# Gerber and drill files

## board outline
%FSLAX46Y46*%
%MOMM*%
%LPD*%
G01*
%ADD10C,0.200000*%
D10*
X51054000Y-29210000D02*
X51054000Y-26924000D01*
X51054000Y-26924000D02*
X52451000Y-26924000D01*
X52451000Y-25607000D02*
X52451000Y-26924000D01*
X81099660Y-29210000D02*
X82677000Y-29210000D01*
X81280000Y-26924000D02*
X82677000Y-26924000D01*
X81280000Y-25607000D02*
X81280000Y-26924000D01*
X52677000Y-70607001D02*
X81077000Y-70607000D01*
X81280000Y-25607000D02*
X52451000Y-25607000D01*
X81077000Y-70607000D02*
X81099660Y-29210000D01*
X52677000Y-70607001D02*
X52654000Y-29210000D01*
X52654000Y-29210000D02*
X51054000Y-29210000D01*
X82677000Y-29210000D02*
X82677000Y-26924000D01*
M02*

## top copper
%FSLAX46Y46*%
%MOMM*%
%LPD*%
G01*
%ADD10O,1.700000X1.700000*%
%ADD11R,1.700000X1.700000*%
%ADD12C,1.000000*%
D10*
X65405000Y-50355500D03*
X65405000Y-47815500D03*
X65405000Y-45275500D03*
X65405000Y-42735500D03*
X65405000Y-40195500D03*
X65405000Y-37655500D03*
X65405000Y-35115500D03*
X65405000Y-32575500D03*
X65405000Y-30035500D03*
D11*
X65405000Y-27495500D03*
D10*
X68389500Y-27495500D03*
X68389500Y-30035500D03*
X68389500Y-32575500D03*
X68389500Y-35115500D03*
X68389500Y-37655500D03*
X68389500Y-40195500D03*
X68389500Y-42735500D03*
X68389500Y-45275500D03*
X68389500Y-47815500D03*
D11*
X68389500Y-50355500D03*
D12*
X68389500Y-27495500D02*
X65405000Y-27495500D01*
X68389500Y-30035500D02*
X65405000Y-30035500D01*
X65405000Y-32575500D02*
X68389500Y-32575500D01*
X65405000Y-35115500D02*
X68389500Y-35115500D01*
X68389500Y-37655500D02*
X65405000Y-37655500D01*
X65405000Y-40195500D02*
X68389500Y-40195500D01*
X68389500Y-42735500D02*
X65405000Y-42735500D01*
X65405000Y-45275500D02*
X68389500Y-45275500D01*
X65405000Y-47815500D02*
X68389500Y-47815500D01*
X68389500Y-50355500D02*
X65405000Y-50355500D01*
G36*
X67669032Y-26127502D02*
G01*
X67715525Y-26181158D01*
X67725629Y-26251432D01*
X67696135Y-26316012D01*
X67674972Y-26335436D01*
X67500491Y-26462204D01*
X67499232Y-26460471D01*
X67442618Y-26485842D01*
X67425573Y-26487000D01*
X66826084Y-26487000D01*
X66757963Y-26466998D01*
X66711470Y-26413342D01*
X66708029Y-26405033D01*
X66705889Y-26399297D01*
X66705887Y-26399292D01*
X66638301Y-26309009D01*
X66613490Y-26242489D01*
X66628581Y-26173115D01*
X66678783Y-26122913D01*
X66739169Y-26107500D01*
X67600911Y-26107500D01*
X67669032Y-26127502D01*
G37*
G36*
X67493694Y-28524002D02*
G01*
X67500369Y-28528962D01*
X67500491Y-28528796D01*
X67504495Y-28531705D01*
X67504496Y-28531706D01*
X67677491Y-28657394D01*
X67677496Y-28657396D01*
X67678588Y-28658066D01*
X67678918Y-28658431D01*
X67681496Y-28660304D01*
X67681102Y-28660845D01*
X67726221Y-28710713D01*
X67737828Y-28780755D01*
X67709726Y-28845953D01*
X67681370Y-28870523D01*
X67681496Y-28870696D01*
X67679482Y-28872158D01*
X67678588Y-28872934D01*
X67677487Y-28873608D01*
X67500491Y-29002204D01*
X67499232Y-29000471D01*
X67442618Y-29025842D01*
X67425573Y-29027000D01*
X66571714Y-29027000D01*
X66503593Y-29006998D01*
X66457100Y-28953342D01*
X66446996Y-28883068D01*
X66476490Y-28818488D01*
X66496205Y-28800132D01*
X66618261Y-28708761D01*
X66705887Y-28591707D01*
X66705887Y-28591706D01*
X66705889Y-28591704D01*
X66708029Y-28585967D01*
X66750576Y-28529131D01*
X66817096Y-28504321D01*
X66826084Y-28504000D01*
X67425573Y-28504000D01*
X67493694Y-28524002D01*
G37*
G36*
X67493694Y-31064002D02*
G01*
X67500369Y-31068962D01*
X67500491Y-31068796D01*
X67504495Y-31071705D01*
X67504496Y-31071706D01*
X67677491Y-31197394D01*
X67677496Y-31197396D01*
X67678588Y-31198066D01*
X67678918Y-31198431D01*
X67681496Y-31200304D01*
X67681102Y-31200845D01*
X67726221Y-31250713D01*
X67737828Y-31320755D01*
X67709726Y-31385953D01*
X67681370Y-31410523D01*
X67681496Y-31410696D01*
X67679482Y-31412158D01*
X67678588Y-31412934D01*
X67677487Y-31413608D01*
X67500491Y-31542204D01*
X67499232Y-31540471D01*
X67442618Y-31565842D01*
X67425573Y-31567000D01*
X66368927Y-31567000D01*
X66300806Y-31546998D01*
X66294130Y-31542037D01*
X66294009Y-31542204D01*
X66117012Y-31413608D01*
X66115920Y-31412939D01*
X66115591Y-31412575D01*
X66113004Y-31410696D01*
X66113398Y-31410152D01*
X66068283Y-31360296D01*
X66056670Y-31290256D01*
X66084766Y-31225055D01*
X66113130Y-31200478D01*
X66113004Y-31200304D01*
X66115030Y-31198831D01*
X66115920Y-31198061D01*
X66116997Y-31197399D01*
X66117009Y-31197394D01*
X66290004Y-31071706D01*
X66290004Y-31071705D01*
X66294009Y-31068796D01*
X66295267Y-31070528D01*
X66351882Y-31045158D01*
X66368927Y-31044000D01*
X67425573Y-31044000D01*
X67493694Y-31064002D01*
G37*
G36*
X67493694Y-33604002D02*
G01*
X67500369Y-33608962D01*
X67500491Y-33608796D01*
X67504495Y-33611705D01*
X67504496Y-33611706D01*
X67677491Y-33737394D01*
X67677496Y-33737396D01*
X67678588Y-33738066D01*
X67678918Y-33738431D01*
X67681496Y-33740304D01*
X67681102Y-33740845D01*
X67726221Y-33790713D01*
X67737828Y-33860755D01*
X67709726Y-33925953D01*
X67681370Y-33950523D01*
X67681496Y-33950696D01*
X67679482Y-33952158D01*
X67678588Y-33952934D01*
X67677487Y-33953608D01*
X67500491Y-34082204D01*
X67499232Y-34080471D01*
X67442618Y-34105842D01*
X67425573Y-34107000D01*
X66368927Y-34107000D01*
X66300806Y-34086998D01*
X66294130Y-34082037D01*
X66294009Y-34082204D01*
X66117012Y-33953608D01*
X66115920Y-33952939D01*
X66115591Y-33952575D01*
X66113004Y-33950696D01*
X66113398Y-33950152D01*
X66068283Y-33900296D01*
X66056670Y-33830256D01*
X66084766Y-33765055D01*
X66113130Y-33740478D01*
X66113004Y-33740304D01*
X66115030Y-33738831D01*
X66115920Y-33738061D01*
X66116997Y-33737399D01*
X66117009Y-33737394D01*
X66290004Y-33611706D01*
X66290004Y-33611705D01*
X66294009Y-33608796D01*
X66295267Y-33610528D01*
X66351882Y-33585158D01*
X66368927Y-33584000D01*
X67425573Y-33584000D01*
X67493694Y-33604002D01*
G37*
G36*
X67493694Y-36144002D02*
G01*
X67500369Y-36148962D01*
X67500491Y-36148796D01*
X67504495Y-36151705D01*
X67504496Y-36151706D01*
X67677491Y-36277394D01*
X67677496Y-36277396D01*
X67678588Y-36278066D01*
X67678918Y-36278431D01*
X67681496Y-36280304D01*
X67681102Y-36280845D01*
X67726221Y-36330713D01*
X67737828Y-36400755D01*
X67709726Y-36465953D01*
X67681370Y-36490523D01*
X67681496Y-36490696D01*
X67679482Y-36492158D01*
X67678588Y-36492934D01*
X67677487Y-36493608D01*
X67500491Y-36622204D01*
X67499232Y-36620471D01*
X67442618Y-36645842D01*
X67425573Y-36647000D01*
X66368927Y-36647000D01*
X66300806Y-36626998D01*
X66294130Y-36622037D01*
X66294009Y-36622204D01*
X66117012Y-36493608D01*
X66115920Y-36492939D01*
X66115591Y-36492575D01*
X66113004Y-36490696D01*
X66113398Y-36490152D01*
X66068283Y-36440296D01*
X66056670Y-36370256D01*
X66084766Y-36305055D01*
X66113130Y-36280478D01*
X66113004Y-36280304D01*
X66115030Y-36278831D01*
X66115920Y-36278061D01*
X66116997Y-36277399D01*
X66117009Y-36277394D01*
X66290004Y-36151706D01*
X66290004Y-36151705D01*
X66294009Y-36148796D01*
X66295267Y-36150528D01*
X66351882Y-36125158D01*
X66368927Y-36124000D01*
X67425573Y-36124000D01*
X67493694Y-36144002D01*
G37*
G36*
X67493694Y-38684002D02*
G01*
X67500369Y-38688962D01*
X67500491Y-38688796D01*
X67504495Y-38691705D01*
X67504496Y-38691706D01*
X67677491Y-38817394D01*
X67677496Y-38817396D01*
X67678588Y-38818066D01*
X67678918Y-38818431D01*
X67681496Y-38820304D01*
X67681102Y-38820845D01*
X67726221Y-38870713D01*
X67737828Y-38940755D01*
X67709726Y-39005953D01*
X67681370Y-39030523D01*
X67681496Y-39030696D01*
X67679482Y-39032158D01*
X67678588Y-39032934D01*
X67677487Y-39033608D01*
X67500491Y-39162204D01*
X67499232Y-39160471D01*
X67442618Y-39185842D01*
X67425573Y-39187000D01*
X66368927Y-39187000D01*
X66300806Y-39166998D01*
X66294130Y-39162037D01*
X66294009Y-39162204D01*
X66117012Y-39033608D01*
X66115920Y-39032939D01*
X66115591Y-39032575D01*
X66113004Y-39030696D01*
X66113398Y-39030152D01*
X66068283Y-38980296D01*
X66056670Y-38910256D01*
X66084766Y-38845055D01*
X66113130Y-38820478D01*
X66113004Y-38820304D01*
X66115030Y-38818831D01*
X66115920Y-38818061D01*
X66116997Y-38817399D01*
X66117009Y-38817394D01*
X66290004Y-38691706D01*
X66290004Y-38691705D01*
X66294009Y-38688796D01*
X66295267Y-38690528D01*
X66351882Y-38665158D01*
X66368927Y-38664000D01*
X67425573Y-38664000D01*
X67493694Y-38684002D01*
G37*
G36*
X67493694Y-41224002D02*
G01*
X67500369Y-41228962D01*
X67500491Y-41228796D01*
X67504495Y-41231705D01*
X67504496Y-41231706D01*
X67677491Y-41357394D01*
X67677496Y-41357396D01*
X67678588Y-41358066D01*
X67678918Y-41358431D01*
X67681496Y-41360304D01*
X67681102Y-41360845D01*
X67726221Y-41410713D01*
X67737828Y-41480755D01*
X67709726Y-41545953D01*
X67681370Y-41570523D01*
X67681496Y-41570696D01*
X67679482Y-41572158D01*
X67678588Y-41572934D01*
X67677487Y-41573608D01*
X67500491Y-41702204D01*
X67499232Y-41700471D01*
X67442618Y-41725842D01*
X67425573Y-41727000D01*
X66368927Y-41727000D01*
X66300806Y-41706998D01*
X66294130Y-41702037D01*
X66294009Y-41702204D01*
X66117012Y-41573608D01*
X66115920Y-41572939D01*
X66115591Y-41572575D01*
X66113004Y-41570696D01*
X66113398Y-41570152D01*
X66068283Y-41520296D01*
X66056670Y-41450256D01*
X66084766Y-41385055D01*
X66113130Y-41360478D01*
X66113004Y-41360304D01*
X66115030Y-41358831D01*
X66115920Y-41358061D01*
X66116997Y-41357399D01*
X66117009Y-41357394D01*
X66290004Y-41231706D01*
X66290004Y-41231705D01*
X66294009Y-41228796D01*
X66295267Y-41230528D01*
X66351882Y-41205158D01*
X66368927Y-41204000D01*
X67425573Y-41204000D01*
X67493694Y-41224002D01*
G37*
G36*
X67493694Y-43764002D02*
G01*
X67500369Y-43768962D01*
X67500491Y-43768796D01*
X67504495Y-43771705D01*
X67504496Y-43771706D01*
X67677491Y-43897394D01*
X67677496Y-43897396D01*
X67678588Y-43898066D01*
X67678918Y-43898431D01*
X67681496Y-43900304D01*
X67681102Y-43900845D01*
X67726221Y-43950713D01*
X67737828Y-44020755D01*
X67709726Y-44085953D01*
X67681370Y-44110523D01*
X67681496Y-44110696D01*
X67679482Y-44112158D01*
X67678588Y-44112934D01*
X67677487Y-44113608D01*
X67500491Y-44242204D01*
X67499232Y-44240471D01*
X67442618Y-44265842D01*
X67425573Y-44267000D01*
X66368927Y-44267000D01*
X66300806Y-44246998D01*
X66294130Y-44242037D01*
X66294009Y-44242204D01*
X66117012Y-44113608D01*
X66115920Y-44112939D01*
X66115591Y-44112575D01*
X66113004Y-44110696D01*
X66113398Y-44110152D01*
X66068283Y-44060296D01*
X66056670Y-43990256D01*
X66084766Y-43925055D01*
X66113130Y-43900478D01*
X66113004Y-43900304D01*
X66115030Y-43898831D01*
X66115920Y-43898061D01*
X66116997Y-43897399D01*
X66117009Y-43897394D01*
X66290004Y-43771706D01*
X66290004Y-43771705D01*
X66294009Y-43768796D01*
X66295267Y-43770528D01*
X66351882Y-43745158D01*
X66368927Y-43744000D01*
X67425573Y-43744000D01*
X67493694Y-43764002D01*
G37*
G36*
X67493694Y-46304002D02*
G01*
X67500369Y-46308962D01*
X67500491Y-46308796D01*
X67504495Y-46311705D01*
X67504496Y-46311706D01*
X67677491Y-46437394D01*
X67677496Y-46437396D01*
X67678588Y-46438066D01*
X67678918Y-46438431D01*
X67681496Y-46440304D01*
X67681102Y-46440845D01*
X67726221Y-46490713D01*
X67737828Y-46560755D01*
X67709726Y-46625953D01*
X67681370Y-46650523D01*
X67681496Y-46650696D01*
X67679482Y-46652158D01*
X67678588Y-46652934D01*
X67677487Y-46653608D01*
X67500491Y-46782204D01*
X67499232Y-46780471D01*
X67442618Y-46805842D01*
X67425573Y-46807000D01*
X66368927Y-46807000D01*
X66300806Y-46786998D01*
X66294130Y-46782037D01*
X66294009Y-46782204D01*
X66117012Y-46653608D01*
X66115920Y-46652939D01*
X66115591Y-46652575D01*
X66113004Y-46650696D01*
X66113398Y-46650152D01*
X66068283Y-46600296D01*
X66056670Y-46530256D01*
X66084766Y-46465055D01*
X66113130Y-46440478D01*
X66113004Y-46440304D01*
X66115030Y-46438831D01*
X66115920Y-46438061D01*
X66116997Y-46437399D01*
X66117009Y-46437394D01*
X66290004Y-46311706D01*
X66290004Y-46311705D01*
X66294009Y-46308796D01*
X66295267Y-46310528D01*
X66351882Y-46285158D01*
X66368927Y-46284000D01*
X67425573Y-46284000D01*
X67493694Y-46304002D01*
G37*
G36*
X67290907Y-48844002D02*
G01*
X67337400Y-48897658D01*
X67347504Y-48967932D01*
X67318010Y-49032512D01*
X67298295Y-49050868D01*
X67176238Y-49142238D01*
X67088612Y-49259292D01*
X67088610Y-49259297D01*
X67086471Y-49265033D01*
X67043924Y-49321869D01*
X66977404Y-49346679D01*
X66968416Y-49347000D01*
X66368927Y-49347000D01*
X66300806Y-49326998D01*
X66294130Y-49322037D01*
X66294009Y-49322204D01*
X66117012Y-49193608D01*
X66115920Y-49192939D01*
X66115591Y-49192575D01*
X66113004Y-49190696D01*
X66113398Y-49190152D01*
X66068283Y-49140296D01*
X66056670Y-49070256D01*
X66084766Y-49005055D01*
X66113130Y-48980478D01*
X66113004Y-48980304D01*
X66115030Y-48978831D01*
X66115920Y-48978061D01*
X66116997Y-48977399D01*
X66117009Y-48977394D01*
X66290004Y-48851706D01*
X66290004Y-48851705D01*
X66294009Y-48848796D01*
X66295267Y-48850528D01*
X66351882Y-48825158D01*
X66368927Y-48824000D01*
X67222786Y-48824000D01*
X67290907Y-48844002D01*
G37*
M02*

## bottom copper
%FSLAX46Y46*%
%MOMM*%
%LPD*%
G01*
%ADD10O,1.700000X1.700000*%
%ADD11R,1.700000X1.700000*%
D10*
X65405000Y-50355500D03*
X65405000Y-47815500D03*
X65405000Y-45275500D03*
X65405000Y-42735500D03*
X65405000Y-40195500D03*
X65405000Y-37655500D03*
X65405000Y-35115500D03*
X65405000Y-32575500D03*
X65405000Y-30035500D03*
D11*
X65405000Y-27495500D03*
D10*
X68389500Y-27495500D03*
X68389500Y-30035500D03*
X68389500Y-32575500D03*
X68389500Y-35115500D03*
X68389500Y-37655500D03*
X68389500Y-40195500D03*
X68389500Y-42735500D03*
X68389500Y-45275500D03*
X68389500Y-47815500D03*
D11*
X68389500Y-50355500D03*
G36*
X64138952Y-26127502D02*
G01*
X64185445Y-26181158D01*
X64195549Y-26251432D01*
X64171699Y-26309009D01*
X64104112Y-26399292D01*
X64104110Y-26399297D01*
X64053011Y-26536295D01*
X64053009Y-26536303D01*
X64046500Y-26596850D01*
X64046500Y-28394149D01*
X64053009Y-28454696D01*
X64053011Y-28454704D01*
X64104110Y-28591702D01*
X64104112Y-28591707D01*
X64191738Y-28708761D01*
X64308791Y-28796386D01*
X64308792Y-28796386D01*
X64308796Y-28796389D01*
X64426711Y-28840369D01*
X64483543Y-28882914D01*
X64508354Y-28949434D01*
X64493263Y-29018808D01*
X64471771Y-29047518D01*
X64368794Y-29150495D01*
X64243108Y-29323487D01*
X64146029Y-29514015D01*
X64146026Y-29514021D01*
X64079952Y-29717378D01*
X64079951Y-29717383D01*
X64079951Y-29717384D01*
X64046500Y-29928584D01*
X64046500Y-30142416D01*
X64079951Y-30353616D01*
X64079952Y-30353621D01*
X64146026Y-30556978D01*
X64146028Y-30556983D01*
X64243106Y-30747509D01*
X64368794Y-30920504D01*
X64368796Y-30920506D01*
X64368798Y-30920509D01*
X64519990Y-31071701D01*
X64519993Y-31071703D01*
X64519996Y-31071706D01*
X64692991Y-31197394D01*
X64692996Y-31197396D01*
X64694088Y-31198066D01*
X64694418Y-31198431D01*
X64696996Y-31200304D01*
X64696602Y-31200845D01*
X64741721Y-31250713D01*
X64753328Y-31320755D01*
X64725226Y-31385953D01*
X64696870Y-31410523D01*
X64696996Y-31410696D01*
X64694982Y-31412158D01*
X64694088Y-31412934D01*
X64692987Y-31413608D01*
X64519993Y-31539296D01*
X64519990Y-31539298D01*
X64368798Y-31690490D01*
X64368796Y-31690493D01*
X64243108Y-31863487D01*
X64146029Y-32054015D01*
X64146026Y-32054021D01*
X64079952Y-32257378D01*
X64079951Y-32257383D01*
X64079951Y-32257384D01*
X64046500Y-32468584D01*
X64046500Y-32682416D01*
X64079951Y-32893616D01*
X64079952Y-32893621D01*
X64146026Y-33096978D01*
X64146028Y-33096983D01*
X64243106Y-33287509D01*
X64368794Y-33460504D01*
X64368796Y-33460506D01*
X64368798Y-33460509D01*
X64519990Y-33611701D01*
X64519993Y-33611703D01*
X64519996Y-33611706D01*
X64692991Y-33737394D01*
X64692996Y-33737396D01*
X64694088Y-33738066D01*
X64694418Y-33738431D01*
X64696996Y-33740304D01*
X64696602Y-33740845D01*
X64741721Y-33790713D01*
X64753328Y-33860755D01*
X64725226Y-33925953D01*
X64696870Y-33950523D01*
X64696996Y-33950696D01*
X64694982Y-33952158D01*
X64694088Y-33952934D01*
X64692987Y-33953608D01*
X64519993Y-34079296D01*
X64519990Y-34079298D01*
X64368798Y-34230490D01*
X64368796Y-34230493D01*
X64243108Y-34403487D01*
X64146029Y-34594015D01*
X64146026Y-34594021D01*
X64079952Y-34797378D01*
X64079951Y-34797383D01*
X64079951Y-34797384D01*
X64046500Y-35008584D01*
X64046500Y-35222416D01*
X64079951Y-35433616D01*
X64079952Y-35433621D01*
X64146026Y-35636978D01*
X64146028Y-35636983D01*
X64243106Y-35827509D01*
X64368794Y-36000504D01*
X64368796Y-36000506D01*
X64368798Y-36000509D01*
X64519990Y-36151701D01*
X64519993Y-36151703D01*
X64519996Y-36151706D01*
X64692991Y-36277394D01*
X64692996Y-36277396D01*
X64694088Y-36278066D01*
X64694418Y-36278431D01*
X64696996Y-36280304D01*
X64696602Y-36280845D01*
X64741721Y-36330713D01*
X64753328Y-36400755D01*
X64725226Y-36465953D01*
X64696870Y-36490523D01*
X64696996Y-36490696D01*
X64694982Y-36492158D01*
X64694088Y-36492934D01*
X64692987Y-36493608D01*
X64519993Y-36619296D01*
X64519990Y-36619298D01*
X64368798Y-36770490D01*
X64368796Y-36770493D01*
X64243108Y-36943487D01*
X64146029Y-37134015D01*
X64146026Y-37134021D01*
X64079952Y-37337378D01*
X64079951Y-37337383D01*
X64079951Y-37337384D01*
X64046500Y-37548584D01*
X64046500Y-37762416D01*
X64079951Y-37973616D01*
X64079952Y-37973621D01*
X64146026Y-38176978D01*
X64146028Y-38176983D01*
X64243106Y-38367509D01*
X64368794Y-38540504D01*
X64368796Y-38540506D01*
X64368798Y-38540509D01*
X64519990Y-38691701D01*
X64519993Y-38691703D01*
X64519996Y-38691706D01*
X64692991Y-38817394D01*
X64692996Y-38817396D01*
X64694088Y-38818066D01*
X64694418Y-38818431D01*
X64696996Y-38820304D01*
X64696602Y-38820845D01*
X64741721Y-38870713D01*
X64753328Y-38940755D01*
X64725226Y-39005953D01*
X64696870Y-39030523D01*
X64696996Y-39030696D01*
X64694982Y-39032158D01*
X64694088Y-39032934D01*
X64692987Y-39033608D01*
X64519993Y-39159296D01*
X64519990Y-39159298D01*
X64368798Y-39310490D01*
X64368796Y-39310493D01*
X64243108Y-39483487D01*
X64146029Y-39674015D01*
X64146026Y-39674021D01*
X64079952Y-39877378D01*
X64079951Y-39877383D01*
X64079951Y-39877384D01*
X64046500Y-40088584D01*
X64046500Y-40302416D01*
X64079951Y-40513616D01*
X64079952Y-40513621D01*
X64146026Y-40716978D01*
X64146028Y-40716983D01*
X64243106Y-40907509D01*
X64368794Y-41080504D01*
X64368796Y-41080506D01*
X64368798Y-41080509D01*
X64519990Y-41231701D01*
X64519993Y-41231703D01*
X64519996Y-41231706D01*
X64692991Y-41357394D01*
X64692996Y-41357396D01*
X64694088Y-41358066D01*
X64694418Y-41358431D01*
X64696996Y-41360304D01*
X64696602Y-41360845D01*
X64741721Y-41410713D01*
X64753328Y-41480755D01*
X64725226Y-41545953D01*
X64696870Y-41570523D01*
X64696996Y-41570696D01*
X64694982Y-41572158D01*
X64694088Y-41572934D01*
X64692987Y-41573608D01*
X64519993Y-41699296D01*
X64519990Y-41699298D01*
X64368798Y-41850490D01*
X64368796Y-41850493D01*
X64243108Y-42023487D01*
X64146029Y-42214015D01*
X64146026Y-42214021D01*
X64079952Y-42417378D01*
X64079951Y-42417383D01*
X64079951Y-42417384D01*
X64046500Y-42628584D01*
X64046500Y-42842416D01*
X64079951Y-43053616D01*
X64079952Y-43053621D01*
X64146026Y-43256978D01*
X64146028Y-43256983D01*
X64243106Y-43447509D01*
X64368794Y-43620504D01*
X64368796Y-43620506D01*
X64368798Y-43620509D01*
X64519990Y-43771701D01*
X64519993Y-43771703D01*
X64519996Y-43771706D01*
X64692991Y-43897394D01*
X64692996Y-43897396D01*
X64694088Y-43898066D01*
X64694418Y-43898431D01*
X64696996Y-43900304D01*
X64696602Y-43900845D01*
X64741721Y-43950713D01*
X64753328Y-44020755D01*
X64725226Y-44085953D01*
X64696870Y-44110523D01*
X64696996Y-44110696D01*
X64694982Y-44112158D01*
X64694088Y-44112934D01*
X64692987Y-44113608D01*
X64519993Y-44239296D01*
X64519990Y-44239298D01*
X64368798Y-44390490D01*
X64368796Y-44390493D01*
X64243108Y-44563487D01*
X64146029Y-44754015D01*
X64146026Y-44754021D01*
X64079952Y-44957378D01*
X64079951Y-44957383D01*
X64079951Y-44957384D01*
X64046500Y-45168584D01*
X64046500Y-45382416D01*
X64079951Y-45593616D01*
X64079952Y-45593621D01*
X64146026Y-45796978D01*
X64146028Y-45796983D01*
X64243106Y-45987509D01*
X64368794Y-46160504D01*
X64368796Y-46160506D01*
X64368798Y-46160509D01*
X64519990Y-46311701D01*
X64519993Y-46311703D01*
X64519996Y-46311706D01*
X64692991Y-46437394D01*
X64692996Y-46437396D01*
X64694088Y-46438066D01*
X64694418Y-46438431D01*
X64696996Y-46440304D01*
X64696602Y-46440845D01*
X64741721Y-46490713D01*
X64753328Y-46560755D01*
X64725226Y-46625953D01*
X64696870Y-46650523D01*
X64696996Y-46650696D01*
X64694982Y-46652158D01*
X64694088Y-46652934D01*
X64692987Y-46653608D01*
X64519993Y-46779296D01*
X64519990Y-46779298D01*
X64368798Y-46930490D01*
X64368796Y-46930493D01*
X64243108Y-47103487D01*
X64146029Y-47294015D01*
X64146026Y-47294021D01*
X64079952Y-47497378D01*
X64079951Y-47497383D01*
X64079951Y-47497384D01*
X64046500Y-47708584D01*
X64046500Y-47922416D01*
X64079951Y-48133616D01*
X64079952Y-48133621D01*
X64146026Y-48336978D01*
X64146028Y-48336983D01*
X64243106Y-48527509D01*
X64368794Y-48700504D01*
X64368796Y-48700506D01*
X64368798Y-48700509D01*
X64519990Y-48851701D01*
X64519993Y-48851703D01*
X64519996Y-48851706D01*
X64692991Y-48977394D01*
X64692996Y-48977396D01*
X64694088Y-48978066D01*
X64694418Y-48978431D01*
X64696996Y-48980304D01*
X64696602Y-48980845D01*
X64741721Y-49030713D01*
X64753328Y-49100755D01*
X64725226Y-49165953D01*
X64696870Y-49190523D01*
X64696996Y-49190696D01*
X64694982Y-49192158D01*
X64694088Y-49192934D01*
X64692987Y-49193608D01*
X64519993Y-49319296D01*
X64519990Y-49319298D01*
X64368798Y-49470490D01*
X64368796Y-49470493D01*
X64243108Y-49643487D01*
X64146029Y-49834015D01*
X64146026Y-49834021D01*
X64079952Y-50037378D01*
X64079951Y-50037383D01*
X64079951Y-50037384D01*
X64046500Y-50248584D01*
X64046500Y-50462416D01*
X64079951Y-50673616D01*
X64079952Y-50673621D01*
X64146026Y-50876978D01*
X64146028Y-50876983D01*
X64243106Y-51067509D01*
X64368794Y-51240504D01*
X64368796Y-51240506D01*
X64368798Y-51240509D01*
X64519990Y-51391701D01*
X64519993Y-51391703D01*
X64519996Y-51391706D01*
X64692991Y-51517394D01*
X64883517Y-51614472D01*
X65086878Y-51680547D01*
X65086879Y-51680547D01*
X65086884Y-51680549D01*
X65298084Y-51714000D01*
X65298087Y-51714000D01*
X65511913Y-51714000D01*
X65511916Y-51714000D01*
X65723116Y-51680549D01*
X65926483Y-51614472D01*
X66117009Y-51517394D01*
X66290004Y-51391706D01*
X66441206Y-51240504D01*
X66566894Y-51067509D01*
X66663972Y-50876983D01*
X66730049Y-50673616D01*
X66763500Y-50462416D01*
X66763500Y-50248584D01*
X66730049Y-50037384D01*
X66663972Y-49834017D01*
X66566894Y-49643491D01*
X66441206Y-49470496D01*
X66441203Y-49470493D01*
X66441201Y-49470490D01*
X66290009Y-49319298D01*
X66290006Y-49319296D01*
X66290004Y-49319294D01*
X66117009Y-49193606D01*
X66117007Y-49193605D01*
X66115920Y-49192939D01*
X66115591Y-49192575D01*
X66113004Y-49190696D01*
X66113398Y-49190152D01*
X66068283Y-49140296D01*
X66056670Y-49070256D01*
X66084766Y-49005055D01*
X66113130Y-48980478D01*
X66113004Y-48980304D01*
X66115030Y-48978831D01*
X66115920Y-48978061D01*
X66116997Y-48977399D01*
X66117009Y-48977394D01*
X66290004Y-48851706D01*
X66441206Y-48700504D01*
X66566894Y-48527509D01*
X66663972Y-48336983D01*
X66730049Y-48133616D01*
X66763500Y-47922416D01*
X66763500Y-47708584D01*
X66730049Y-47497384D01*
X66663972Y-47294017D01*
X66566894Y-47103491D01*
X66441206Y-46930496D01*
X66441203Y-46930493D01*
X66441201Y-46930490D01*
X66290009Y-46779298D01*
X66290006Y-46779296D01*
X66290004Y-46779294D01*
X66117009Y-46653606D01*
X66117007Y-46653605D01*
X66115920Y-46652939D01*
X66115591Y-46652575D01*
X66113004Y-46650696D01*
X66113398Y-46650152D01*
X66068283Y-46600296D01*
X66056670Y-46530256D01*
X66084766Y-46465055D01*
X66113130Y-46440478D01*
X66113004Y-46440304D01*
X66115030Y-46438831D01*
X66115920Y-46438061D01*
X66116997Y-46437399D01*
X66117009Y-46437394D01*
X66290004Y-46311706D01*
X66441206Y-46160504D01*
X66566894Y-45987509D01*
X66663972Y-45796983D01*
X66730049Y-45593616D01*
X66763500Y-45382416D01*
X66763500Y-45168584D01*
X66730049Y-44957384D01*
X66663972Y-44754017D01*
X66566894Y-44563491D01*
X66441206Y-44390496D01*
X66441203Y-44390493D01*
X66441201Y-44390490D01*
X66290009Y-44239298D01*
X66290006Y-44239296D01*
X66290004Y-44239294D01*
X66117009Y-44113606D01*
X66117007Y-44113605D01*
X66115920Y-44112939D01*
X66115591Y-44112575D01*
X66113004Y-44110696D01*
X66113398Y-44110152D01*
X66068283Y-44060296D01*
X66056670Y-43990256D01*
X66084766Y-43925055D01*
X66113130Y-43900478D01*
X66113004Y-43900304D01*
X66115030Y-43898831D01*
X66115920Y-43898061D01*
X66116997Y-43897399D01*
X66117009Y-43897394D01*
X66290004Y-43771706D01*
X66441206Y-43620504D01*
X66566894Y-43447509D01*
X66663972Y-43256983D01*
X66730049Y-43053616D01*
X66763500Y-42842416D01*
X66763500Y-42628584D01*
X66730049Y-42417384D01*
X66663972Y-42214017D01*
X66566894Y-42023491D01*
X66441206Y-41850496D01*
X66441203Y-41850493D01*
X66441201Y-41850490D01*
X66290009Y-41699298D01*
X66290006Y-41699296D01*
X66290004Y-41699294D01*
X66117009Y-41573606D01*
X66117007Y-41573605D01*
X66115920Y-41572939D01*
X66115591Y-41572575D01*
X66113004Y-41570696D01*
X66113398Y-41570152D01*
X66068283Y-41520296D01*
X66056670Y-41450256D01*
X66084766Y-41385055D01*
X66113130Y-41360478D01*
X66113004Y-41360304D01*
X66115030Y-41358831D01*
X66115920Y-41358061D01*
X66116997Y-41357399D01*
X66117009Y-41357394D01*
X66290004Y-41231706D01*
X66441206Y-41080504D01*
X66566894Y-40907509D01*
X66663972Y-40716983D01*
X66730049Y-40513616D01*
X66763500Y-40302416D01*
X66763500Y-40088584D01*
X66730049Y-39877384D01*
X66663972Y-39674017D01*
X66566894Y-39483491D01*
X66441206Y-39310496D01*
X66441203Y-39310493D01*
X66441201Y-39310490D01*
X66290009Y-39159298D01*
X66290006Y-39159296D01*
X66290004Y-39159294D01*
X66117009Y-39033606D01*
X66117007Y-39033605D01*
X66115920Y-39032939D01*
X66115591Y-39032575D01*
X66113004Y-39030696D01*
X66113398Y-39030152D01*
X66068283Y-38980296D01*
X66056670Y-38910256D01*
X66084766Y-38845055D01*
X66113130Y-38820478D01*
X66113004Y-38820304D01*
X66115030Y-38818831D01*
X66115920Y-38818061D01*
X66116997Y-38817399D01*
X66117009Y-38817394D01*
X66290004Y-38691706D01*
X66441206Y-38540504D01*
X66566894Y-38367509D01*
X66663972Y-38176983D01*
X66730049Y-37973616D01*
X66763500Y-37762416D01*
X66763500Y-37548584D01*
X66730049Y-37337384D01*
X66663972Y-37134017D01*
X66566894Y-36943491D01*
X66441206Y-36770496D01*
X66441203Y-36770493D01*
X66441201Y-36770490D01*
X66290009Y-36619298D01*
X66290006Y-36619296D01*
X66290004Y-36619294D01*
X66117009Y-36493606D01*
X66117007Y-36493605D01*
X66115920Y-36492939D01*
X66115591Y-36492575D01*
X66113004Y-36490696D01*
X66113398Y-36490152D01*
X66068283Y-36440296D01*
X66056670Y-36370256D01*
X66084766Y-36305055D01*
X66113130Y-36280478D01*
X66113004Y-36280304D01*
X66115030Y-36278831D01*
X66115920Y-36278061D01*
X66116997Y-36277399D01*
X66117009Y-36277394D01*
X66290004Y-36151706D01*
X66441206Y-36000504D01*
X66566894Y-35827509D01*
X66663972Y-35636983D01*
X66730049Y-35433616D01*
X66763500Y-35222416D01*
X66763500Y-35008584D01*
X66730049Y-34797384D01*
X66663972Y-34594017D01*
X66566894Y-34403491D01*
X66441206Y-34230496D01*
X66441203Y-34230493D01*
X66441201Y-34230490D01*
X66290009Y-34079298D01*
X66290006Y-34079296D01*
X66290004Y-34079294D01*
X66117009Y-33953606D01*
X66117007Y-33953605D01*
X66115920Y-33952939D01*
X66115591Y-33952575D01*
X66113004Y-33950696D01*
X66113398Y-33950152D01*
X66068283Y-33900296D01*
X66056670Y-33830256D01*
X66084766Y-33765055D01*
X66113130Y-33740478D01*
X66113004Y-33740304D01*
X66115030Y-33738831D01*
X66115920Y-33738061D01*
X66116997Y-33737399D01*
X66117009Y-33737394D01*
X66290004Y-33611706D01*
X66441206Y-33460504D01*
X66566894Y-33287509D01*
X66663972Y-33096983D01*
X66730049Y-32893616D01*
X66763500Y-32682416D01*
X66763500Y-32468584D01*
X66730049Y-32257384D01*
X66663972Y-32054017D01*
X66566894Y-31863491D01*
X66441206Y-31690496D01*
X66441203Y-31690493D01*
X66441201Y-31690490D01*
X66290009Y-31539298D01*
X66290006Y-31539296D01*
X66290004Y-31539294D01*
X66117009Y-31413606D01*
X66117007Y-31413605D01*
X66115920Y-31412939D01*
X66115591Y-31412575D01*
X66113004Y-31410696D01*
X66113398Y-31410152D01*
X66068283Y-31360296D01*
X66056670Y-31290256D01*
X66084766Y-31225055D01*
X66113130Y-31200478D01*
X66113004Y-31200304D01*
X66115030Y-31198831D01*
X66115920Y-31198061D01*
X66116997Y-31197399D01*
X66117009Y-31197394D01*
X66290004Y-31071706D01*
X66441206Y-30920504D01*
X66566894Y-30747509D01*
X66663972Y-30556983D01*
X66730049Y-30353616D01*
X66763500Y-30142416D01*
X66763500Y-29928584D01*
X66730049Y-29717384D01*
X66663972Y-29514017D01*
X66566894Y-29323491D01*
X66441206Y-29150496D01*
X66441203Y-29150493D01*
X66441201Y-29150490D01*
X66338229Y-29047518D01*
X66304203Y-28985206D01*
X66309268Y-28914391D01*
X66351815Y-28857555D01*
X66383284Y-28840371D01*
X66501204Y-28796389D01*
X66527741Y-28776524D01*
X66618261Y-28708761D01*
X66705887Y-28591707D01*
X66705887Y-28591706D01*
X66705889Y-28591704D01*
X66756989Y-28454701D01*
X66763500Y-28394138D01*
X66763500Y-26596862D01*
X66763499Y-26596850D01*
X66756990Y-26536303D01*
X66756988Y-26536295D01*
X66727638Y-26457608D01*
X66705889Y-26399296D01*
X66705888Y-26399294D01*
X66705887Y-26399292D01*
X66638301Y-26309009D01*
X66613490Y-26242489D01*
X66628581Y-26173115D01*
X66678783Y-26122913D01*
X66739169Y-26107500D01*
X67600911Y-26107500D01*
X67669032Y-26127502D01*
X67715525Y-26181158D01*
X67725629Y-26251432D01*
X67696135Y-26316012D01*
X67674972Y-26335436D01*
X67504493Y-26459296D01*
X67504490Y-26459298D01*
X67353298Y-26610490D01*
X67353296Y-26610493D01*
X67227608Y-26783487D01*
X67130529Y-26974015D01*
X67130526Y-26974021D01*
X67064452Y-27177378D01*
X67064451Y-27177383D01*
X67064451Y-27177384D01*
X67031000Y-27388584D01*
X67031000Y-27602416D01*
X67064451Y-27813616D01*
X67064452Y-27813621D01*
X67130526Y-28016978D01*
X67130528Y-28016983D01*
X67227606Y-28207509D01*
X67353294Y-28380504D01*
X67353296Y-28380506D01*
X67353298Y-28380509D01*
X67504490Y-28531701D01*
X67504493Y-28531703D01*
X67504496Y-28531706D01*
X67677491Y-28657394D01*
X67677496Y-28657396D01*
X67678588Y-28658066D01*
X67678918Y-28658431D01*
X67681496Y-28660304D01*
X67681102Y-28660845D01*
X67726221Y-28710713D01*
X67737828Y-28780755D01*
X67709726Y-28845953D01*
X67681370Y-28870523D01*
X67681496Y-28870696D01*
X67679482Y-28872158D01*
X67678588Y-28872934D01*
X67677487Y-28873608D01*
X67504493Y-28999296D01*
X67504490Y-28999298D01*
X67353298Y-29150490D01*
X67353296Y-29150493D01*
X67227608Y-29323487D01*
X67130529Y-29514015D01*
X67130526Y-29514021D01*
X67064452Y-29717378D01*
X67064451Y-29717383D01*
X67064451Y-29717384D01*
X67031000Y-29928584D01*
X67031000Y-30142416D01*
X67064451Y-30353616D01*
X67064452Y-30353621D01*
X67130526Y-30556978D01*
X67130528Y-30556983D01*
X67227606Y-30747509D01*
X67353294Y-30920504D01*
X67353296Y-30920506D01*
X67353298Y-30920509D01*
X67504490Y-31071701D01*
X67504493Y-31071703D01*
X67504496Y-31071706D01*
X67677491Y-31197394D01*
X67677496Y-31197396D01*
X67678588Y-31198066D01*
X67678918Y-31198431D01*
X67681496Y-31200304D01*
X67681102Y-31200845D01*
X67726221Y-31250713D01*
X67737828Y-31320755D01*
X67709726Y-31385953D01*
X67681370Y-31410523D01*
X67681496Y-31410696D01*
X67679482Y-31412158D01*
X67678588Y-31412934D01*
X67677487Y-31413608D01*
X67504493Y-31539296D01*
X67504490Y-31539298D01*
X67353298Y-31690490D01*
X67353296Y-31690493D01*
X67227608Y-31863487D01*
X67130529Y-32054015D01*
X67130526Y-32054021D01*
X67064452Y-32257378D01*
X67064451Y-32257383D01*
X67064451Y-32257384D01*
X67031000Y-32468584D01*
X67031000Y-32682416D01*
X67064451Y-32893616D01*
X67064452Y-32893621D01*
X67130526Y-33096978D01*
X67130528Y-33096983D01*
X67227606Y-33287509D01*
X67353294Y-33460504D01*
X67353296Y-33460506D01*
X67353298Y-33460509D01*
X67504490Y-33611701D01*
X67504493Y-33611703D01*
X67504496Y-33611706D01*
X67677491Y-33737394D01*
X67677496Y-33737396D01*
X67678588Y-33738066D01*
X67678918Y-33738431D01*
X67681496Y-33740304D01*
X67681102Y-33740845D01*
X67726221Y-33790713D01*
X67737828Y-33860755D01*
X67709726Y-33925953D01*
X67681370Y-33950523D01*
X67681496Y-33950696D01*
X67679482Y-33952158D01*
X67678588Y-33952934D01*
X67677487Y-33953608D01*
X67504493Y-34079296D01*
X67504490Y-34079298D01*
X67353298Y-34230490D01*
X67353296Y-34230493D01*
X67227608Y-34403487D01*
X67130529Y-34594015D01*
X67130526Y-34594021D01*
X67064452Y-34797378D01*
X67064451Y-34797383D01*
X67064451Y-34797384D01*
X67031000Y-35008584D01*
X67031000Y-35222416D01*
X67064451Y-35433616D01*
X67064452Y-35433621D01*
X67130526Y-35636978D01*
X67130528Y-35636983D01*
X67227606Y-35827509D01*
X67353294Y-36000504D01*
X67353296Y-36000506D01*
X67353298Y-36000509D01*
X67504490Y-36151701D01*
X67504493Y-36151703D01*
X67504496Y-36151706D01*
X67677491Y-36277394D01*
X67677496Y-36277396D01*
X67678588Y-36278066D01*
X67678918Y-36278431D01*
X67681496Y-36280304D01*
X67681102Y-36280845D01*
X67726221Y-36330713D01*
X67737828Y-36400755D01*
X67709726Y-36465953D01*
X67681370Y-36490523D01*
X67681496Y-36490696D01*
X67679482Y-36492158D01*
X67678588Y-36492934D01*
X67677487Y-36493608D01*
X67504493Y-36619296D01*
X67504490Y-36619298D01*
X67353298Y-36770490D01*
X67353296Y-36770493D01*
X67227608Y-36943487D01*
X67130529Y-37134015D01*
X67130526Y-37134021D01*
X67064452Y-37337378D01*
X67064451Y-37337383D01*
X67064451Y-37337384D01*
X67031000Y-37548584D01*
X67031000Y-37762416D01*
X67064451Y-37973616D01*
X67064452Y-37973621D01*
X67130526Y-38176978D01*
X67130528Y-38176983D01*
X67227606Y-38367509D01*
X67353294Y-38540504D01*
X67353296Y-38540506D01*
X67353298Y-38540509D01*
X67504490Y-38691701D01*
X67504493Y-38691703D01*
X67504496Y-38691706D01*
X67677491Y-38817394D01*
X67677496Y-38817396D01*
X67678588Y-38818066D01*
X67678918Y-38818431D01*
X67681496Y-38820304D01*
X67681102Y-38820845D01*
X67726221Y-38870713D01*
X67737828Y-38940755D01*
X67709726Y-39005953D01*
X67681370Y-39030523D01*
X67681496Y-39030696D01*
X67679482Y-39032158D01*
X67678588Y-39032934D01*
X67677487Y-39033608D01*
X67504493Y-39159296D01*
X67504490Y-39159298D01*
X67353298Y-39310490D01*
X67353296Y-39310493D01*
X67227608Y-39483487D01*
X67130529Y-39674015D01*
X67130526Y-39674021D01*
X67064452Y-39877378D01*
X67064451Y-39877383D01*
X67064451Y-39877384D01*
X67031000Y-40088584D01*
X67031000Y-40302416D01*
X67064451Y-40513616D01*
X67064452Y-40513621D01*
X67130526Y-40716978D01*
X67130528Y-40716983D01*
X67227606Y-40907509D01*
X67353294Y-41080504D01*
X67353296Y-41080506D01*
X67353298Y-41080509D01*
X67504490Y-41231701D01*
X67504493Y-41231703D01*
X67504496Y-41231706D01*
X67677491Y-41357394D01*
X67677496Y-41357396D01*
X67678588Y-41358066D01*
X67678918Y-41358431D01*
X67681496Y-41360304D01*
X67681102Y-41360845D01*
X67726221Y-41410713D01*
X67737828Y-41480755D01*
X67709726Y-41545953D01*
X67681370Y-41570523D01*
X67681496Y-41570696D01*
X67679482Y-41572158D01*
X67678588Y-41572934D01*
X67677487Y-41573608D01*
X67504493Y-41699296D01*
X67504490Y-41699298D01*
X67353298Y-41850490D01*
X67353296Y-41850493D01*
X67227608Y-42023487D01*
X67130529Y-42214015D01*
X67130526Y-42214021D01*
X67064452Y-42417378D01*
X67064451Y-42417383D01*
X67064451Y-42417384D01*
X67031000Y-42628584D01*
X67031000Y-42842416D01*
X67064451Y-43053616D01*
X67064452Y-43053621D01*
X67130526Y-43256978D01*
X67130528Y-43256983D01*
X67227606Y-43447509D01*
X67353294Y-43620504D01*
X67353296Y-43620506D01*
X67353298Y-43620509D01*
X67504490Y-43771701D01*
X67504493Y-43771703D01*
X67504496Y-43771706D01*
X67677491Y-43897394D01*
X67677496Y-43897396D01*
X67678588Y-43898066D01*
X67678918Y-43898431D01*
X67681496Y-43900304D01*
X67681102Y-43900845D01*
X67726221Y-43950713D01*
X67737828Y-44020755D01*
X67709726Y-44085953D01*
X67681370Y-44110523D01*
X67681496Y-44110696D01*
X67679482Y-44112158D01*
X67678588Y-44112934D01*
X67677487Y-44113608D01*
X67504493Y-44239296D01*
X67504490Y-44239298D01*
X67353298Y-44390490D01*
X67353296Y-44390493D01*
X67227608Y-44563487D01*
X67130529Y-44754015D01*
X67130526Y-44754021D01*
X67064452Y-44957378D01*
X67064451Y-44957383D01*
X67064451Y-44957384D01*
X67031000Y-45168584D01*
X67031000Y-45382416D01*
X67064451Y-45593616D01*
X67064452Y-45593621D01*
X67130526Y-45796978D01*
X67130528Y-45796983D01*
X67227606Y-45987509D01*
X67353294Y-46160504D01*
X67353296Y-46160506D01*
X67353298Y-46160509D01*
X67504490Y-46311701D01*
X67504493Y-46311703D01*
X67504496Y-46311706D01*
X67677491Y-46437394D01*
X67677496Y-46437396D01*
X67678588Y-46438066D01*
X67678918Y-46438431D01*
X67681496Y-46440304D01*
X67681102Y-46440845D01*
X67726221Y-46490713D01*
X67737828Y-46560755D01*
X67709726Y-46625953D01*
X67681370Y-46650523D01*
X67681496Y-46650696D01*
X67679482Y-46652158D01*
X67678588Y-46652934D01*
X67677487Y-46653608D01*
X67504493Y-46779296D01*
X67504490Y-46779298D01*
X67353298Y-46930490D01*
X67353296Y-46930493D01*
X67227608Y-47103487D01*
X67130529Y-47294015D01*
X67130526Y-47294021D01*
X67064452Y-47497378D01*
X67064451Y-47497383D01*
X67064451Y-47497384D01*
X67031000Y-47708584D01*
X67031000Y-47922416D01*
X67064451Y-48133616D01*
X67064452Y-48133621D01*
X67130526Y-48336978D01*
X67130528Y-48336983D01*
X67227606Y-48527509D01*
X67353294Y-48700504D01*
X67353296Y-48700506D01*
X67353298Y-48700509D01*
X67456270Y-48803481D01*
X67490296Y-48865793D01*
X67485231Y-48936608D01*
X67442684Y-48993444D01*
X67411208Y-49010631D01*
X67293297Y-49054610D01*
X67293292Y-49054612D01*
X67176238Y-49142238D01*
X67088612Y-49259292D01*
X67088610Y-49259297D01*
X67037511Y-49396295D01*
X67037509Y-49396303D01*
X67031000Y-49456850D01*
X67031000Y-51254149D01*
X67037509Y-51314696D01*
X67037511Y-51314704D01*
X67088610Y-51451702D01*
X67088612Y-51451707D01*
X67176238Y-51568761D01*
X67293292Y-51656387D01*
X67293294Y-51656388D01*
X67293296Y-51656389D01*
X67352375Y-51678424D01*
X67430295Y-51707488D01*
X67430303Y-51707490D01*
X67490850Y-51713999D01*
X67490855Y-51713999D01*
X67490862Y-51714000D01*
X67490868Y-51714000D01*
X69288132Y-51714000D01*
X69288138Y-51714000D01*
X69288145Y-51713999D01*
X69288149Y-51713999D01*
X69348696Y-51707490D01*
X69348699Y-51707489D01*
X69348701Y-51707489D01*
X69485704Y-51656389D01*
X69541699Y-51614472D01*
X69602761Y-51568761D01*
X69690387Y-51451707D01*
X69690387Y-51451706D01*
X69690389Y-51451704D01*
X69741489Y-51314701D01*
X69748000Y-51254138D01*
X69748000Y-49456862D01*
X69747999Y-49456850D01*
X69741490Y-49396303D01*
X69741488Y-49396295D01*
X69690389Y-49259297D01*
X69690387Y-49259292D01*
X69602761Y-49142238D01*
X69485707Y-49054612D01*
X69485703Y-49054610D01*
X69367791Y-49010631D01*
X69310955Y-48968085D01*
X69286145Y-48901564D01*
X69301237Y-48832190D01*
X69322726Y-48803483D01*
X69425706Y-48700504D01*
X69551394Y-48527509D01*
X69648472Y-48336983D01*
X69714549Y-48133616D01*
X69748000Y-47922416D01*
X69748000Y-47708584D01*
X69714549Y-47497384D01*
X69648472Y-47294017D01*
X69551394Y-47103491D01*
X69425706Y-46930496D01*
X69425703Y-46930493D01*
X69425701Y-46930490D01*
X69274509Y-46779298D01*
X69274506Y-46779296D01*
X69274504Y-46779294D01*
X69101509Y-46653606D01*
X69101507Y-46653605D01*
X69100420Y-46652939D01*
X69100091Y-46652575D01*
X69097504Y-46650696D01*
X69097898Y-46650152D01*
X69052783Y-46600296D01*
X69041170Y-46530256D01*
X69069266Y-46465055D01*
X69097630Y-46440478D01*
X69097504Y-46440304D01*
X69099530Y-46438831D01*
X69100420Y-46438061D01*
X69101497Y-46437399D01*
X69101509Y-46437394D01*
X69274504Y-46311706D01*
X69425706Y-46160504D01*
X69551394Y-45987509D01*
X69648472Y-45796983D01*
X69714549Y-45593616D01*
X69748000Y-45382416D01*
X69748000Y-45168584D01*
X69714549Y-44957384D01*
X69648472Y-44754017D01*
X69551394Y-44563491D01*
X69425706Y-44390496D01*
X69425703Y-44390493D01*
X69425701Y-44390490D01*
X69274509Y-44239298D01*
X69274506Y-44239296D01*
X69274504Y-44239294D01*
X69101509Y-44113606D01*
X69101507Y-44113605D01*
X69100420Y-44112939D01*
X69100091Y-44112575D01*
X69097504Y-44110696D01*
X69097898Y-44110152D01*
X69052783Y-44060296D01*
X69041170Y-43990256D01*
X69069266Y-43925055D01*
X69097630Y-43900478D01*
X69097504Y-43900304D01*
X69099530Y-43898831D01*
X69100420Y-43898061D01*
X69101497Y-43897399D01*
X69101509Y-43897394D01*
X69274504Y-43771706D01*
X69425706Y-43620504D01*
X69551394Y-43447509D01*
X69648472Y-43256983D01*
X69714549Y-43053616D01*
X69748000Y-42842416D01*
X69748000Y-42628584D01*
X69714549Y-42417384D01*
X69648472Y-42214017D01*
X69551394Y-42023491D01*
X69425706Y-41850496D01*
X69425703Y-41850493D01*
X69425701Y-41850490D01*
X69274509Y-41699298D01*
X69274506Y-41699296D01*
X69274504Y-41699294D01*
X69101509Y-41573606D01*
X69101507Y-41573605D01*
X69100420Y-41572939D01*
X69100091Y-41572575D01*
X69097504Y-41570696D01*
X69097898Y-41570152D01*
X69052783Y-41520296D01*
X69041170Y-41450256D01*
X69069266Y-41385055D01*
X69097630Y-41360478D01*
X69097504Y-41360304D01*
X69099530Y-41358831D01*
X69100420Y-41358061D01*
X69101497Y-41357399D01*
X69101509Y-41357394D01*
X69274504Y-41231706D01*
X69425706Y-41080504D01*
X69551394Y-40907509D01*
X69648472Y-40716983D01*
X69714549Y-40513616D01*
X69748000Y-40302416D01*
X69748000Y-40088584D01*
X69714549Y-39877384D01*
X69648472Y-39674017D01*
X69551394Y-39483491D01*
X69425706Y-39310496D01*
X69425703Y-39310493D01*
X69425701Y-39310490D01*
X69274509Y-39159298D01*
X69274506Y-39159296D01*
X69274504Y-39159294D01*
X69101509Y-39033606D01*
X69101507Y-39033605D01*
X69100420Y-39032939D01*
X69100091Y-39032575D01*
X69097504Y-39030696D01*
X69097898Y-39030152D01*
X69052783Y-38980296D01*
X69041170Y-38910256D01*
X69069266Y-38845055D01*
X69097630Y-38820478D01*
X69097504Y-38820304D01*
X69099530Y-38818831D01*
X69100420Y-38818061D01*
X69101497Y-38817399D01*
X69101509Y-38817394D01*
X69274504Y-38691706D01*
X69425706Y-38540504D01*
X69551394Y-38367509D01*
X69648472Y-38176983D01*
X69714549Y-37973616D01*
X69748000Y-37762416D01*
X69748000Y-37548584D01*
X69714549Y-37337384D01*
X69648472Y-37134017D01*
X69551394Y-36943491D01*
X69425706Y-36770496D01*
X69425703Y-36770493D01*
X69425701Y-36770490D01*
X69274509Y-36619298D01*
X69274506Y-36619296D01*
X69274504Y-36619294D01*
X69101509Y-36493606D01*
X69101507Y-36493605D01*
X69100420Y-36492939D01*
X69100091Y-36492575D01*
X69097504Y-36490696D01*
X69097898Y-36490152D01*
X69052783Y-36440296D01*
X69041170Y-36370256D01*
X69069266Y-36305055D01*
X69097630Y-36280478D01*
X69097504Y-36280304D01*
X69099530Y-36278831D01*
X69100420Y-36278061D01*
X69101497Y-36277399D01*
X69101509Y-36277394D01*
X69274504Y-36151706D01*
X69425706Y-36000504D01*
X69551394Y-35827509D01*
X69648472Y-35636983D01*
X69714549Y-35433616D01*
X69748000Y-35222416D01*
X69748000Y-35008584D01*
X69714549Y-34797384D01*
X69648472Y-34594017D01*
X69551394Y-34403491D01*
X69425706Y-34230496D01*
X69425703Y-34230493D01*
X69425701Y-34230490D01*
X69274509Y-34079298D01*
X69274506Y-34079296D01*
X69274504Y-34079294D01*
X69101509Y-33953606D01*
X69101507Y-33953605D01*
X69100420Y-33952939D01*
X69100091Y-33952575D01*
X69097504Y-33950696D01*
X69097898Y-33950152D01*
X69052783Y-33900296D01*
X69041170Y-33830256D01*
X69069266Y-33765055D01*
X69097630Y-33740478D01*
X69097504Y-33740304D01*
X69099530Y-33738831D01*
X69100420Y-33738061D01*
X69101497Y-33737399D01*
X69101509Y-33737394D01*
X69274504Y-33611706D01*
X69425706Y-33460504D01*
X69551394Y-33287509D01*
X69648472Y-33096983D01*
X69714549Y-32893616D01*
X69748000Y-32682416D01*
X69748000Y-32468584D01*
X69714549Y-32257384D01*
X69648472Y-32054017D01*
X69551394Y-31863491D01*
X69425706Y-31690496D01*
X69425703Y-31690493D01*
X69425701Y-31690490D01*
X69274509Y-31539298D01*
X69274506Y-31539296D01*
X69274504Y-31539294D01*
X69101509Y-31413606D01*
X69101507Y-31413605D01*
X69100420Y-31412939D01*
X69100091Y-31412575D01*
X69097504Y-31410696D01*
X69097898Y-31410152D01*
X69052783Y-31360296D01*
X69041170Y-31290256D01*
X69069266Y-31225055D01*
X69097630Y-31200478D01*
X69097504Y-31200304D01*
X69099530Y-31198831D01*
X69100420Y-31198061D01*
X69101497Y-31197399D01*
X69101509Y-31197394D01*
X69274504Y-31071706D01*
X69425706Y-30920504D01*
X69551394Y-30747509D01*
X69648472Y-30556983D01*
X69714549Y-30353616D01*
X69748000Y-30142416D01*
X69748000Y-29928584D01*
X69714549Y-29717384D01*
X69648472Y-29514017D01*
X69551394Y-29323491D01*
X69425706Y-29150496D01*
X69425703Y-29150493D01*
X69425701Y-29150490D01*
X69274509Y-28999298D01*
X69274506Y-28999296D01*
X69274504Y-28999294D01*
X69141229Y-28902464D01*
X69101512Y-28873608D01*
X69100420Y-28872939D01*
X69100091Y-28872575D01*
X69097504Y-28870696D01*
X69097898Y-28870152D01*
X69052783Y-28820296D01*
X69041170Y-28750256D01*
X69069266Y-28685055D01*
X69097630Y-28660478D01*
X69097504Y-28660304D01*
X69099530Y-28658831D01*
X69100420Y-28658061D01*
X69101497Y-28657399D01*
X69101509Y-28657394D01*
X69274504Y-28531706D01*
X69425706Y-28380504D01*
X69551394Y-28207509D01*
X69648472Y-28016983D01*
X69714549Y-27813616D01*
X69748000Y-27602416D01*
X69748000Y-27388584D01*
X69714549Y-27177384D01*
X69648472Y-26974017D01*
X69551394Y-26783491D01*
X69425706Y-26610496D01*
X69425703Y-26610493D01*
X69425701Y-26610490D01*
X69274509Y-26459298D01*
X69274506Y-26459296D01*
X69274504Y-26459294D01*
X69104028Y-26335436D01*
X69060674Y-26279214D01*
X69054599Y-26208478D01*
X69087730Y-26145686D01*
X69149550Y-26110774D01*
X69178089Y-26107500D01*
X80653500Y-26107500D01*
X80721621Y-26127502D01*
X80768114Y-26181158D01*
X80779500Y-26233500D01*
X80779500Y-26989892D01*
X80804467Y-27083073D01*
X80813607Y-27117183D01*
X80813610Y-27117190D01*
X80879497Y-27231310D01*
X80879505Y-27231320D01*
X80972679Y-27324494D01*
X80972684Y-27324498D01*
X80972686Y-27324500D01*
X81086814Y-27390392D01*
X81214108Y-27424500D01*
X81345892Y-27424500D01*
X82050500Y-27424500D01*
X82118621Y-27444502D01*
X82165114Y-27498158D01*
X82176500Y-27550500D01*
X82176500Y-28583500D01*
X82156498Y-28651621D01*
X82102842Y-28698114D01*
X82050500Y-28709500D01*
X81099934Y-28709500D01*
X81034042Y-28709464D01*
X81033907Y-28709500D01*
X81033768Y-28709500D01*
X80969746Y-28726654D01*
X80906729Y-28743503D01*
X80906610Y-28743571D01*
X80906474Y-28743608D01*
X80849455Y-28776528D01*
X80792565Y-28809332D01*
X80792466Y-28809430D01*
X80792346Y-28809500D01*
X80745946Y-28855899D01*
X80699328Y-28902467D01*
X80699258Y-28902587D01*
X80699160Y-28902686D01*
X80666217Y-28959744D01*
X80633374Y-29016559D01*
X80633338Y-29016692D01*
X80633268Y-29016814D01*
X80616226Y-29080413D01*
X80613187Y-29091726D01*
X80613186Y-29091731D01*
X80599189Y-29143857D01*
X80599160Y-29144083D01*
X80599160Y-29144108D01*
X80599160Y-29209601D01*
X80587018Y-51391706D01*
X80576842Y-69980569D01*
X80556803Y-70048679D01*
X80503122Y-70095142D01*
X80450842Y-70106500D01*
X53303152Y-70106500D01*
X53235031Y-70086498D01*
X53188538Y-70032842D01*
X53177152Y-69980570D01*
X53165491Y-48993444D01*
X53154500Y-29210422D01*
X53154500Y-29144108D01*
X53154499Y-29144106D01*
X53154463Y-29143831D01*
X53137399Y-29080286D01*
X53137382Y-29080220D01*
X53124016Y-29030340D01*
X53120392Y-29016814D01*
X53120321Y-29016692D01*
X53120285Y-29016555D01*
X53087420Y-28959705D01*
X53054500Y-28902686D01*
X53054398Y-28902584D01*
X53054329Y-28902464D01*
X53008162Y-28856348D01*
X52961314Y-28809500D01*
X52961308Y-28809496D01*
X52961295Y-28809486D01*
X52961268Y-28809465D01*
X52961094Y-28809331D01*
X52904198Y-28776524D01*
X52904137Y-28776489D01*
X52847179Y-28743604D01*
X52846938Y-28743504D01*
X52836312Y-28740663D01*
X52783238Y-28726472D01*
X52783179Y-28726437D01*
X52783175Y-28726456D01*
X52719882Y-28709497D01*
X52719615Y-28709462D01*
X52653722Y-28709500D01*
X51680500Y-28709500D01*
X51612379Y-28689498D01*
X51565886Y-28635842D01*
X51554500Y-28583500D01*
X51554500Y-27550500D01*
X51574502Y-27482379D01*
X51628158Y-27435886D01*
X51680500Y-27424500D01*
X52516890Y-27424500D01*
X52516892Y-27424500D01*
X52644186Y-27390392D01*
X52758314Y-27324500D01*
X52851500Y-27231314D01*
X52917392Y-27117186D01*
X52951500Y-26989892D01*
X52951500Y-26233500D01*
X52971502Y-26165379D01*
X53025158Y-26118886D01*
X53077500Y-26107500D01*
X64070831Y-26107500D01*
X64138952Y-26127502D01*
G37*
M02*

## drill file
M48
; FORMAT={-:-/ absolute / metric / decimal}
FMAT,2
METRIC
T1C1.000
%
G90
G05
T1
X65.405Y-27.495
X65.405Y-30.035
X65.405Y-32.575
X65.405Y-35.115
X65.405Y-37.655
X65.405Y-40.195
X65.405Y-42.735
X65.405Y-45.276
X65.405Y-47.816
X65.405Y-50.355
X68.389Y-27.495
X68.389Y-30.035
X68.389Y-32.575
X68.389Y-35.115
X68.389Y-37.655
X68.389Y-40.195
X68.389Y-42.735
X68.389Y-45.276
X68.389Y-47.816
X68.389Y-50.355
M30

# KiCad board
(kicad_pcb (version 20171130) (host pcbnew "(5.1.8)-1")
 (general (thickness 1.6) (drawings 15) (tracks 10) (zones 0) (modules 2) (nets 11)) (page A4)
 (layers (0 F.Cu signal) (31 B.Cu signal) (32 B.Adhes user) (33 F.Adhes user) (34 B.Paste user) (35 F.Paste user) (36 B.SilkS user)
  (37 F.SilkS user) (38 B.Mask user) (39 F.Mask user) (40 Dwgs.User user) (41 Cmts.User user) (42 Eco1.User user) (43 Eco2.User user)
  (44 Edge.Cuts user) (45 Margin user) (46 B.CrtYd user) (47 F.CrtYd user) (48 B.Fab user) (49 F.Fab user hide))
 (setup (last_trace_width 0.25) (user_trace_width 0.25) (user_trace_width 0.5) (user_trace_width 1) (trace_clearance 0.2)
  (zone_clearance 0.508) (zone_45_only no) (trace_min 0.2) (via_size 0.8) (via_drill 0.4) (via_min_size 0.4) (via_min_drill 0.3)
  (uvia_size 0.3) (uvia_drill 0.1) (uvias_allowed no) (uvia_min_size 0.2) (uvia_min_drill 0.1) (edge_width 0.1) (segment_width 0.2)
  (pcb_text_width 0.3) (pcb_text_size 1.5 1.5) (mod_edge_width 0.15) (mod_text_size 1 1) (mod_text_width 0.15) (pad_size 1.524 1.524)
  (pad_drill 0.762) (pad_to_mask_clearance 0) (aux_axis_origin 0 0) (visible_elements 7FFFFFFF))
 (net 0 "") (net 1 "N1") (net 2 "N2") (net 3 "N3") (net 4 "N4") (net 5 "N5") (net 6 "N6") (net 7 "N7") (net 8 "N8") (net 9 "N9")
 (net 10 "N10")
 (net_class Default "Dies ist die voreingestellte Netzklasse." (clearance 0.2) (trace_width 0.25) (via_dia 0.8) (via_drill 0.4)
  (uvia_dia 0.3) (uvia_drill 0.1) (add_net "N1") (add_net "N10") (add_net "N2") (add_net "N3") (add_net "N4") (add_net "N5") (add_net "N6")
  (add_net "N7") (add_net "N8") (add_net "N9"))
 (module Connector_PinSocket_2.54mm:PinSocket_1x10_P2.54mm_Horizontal (layer F.Cu) (at 65.405 27.4955)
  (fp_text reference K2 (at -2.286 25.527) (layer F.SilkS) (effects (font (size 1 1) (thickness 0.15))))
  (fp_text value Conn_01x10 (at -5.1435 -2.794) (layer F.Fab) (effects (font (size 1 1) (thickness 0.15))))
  (pad 10 thru_hole oval (at 0 22.86) (size 1.7 1.7) (drill 1) (layers *.Cu *.Mask) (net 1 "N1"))
  (pad 9 thru_hole oval (at 0 20.32) (size 1.7 1.7) (drill 1) (layers *.Cu *.Mask) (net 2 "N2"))
  (pad 8 thru_hole oval (at 0 17.78) (size 1.7 1.7) (drill 1) (layers *.Cu *.Mask) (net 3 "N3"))
  (pad 7 thru_hole oval (at 0 15.24) (size 1.7 1.7) (drill 1) (layers *.Cu *.Mask) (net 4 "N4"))
  (pad 6 thru_hole oval (at 0 12.7) (size 1.7 1.7) (drill 1) (layers *.Cu *.Mask) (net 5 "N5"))
  (pad 5 thru_hole oval (at 0 10.16) (size 1.7 1.7) (drill 1) (layers *.Cu *.Mask) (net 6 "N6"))
  (pad 4 thru_hole oval (at 0 7.62) (size 1.7 1.7) (drill 1) (layers *.Cu *.Mask) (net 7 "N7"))
  (pad 3 thru_hole oval (at 0 5.08) (size 1.7 1.7) (drill 1) (layers *.Cu *.Mask) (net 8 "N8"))
  (pad 2 thru_hole oval (at 0 2.54) (size 1.7 1.7) (drill 1) (layers *.Cu *.Mask) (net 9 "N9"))
  (pad 1 thru_hole rect (at 0 0) (size 1.7 1.7) (drill 1) (layers *.Cu *.Mask) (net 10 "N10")))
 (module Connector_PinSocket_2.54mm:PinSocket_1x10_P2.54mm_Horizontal (layer F.Cu) (at 68.3895 50.3555 180)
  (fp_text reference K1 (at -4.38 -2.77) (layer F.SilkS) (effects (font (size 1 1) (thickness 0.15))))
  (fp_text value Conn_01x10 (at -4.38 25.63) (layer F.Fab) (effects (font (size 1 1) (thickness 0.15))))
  (pad 10 thru_hole oval (at 0 22.86 180) (size 1.7 1.7) (drill 1) (layers *.Cu *.Mask) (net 10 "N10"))
  (pad 9 thru_hole oval (at 0 20.32 180) (size 1.7 1.7) (drill 1) (layers *.Cu *.Mask) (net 9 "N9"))
  (pad 8 thru_hole oval (at 0 17.78 180) (size 1.7 1.7) (drill 1) (layers *.Cu *.Mask) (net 8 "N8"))
  (pad 7 thru_hole oval (at 0 15.24 180) (size 1.7 1.7) (drill 1) (layers *.Cu *.Mask) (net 7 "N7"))
  (pad 6 thru_hole oval (at 0 12.7 180) (size 1.7 1.7) (drill 1) (layers *.Cu *.Mask) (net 6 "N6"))
  (pad 5 thru_hole oval (at 0 10.16 180) (size 1.7 1.7) (drill 1) (layers *.Cu *.Mask) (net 5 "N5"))
  (pad 4 thru_hole oval (at 0 7.62 180) (size 1.7 1.7) (drill 1) (layers *.Cu *.Mask) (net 4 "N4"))
  (pad 3 thru_hole oval (at 0 5.08 180) (size 1.7 1.7) (drill 1) (layers *.Cu *.Mask) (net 3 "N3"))
  (pad 2 thru_hole oval (at 0 2.54 180) (size 1.7 1.7) (drill 1) (layers *.Cu *.Mask) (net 2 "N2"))
  (pad 1 thru_hole rect (at 0 0 180) (size 1.7 1.7) (drill 1) (layers *.Cu *.Mask) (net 1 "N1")))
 (gr_line (start 51.054 29.21) (end 51.054 26.924) (layer Edge.Cuts) (width 0.2))
 (gr_line (start 51.054 26.924) (end 52.451 26.924) (layer Edge.Cuts) (width 0.2))
 (gr_line (start 52.451 25.607) (end 52.451 26.924) (layer Edge.Cuts) (width 0.2))
 (gr_line (start 81.09966 29.21) (end 82.677 29.21) (layer Edge.Cuts) (width 0.2))
 (gr_line (start 81.28 26.924) (end 82.677 26.924) (layer Edge.Cuts) (width 0.2))
 (gr_line (start 81.28 25.607) (end 81.28 26.924) (layer Edge.Cuts) (width 0.2))
 (gr_line (start 52.677 70.607001) (end 81.077 70.607) (layer Edge.Cuts) (width 0.2))
 (gr_line (start 81.28 25.607) (end 52.451 25.607) (layer Edge.Cuts) (width 0.2))
 (gr_line (start 81.077 70.607) (end 81.09966 29.21) (layer Edge.Cuts) (width 0.2))
 (gr_line (start 52.677 70.607001) (end 52.654 29.21) (layer Edge.Cuts) (width 0.2))
 (gr_line (start 52.654 29.21) (end 51.054 29.21) (layer Edge.Cuts) (width 0.2))
 (gr_line (start 82.677 29.21) (end 82.677 26.924) (layer Edge.Cuts) (width 0.2))
 (segment (start 68.3895 27.4955) (end 65.405 27.4955) (width 1) (layer F.Cu) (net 10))
 (segment (start 68.3895 30.0355) (end 65.405 30.0355) (width 1) (layer F.Cu) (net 9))
 (segment (start 65.405 32.5755) (end 68.3895 32.5755) (width 1) (layer F.Cu) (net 8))
 (segment (start 65.405 35.1155) (end 68.3895 35.1155) (width 1) (layer F.Cu) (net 7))
 (segment (start 68.3895 37.6555) (end 65.405 37.6555) (width 1) (layer F.Cu) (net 6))
 (segment (start 65.405 40.1955) (end 68.3895 40.1955) (width 1) (layer F.Cu) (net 5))
 (segment (start 68.3895 42.7355) (end 65.405 42.7355) (width 1) (layer F.Cu) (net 4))
 (segment (start 65.405 45.2755) (end 68.3895 45.2755) (width 1) (layer F.Cu) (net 3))
 (segment (start 65.405 47.8155) (end 68.3895 47.8155) (width 1) (layer F.Cu) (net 2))
 (segment (start 68.3895 50.3555) (end 65.405 50.3555) (width 1) (layer F.Cu) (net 1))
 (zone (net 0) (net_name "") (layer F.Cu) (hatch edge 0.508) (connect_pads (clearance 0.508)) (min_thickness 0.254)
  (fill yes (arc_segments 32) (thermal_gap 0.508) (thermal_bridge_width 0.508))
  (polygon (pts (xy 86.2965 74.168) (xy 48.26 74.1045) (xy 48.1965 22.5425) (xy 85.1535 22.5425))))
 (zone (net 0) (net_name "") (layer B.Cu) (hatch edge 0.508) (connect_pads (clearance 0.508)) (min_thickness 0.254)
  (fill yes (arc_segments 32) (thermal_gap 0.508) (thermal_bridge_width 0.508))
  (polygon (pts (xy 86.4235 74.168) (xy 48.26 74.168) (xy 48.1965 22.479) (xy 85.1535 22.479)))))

